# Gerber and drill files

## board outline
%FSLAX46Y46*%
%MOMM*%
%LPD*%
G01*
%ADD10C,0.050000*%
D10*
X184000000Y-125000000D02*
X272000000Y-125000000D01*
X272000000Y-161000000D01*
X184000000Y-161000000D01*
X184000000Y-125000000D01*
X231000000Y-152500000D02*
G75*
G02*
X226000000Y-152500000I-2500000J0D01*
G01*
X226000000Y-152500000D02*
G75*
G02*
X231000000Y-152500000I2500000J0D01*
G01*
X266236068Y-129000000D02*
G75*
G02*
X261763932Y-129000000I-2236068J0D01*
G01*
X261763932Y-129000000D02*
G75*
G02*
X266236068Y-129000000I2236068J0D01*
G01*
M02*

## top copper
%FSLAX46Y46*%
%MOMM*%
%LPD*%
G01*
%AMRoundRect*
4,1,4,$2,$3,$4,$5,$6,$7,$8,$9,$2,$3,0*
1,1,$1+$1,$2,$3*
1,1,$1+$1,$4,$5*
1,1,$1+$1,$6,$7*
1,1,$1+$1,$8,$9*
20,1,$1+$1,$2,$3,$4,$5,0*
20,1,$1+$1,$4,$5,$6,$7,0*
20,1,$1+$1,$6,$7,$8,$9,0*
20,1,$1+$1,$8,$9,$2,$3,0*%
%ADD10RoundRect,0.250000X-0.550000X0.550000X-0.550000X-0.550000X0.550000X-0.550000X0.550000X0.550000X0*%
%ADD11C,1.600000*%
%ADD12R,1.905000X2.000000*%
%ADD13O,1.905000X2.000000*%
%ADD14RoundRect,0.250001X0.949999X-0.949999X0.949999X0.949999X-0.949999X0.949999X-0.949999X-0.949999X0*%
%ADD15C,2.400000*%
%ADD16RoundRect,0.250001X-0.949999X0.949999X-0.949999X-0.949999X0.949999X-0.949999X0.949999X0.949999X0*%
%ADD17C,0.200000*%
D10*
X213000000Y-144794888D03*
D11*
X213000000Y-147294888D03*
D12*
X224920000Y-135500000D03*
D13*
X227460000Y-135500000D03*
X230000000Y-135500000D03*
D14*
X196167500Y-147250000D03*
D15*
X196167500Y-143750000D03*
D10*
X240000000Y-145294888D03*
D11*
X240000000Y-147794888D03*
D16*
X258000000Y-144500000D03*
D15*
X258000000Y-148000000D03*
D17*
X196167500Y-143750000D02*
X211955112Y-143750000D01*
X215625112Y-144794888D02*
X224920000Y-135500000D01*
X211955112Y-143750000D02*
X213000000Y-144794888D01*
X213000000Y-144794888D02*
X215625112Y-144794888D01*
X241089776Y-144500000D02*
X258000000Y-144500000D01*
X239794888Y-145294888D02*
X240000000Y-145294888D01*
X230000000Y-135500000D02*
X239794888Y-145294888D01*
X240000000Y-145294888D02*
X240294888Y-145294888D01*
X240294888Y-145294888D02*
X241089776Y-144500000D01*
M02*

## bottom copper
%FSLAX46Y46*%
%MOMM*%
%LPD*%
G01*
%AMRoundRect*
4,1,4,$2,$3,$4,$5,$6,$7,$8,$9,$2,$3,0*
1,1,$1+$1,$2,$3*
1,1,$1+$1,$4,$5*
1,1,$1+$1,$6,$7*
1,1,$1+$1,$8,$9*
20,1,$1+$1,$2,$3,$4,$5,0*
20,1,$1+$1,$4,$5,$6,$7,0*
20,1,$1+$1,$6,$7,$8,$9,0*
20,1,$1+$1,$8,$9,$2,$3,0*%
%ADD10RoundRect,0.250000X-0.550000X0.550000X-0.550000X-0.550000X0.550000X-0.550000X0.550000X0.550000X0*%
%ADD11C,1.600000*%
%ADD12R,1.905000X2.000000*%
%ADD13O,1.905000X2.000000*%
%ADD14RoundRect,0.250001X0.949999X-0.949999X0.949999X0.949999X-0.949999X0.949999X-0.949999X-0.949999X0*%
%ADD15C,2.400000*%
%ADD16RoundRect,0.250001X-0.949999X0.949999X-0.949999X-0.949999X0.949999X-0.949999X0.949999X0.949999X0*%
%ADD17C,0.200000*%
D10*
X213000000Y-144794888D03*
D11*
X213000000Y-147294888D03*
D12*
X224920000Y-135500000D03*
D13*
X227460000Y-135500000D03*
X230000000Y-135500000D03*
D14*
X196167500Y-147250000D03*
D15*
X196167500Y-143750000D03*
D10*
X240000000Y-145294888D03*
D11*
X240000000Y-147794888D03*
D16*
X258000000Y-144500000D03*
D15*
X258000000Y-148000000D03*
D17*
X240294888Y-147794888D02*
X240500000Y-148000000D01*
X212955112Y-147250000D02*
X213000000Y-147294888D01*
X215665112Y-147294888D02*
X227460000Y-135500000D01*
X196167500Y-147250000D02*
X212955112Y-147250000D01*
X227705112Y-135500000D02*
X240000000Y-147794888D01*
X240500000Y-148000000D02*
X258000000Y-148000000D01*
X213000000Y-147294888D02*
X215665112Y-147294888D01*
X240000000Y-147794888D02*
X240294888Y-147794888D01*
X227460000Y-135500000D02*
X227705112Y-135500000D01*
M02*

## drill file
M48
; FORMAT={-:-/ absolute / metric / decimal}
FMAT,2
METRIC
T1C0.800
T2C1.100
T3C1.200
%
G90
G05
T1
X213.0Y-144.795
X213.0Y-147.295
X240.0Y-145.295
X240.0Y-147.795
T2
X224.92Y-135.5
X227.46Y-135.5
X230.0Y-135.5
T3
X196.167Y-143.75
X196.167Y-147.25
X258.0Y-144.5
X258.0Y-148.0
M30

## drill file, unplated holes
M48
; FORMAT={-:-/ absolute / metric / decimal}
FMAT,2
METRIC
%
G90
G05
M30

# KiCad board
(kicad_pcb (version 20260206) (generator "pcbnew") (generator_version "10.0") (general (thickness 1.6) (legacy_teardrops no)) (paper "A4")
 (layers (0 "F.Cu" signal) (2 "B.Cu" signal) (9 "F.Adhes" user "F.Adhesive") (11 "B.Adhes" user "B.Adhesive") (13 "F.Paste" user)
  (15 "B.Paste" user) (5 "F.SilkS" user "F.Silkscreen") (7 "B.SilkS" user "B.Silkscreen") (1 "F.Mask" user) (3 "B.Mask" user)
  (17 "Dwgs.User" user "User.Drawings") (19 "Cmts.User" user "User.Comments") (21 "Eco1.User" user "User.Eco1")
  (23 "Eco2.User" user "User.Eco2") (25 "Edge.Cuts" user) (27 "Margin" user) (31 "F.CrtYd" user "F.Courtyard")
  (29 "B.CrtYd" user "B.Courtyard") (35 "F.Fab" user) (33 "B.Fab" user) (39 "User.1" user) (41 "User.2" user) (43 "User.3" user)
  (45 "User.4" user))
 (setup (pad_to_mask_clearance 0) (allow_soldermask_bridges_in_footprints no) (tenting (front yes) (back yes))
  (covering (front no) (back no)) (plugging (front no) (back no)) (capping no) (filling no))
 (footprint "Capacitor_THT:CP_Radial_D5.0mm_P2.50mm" (layer "F.Cu") (at 213 144.794888 -90)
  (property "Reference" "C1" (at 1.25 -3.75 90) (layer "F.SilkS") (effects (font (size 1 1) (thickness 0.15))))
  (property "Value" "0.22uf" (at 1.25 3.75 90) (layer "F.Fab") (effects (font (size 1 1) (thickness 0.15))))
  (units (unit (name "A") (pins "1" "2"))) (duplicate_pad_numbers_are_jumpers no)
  (pad "1" thru_hole roundrect (at 0 0 270) (size 1.6 1.6) (drill 0.8) (layers "*.Cu" "*.Mask") (remove_unused_layers no)
   (roundrect_rratio 0.15625) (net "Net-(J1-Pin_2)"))
  (pad "2" thru_hole circle (at 2.5 0 270) (size 1.6 1.6) (drill 0.8) (layers "*.Cu" "*.Mask") (remove_unused_layers no) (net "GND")))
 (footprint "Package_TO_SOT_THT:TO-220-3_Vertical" (layer "F.Cu") (at 224.92 135.5)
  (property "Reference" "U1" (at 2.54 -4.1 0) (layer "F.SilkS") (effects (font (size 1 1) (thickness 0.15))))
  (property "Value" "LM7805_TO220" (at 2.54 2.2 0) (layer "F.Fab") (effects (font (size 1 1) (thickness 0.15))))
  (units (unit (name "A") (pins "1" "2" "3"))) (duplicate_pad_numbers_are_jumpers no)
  (pad "1" thru_hole rect (at 0 0) (size 1.905 2) (drill 1.1) (layers "*.Cu" "*.Mask") (remove_unused_layers no) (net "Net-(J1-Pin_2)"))
  (pad "2" thru_hole oval (at 2.54 0) (size 1.905 2) (drill 1.1) (layers "*.Cu" "*.Mask") (remove_unused_layers no) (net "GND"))
  (pad "3" thru_hole oval (at 5.08 0) (size 1.905 2) (drill 1.1) (layers "*.Cu" "*.Mask") (remove_unused_layers no) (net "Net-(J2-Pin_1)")))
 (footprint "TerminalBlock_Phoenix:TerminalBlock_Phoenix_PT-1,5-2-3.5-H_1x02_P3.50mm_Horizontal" (layer "F.Cu") (at 196.1675 147.25 90)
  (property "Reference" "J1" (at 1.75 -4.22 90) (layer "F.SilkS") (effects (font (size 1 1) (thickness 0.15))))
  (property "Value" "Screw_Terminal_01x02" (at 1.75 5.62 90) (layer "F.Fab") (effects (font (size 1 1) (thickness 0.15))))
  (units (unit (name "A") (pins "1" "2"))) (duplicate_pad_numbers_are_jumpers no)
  (pad "1" thru_hole roundrect (at 0 0 90) (size 2.4 2.4) (drill 1.2) (layers "*.Cu" "*.Mask") (remove_unused_layers no)
   (roundrect_rratio 0.104167) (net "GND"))
  (pad "2" thru_hole circle (at 3.5 0 90) (size 2.4 2.4) (drill 1.2) (layers "*.Cu" "*.Mask") (remove_unused_layers no)
   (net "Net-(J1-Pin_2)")))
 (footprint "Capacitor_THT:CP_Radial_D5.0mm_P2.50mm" (layer "F.Cu") (at 240 145.294888 -90)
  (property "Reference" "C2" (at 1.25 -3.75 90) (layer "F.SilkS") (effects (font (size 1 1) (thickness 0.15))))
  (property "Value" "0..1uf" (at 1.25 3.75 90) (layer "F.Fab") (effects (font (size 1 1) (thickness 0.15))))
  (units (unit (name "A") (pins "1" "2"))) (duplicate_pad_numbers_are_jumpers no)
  (pad "1" thru_hole roundrect (at 0 0 270) (size 1.6 1.6) (drill 0.8) (layers "*.Cu" "*.Mask") (remove_unused_layers no)
   (roundrect_rratio 0.15625) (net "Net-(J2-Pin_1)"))
  (pad "2" thru_hole circle (at 2.5 0 270) (size 1.6 1.6) (drill 0.8) (layers "*.Cu" "*.Mask") (remove_unused_layers no) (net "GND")))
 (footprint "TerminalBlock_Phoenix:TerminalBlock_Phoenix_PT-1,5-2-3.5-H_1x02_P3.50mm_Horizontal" (layer "F.Cu") (at 258 144.5 -90)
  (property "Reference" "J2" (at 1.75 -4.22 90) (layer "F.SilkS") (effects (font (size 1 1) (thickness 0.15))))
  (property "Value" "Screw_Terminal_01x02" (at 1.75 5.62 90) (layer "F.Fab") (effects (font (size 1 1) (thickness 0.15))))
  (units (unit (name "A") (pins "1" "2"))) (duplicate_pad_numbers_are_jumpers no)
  (pad "1" thru_hole roundrect (at 0 0 270) (size 2.4 2.4) (drill 1.2) (layers "*.Cu" "*.Mask") (remove_unused_layers no)
   (roundrect_rratio 0.104167) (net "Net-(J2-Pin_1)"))
  (pad "2" thru_hole circle (at 3.5 0 270) (size 2.4 2.4) (drill 1.2) (layers "*.Cu" "*.Mask") (remove_unused_layers no) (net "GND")))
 (gr_rect (start 184 125) (end 272 161) (stroke (width 0.05) (type default)) (fill no) (layer "Edge.Cuts"))
 (gr_circle (center 228.5 152.5) (end 227 154.5) (stroke (width 0.05) (type default)) (fill no) (layer "Edge.Cuts"))
 (gr_circle (center 264 129) (end 263 131) (stroke (width 0.05) (type default)) (fill no) (layer "Edge.Cuts"))
 (segment (start 196.1675 143.75) (end 211.955112 143.75) (width 0.2) (layer "F.Cu") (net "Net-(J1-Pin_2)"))
 (segment (start 215.625112 144.794888) (end 224.92 135.5) (width 0.2) (layer "F.Cu") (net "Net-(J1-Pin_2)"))
 (segment (start 211.955112 143.75) (end 213 144.794888) (width 0.2) (layer "F.Cu") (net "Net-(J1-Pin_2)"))
 (segment (start 213 144.794888) (end 215.625112 144.794888) (width 0.2) (layer "F.Cu") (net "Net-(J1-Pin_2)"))
 (segment (start 240.294888 147.794888) (end 240.5 148) (width 0.2) (layer "B.Cu") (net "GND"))
 (segment (start 212.955112 147.25) (end 213 147.294888) (width 0.2) (layer "B.Cu") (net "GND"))
 (segment (start 215.665112 147.294888) (end 227.46 135.5) (width 0.2) (layer "B.Cu") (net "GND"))
 (segment (start 196.1675 147.25) (end 212.955112 147.25) (width 0.2) (layer "B.Cu") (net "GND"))
 (segment (start 227.705112 135.5) (end 240 147.794888) (width 0.2) (layer "B.Cu") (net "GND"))
 (segment (start 240.5 148) (end 258 148) (width 0.2) (layer "B.Cu") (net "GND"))
 (segment (start 213 147.294888) (end 215.665112 147.294888) (width 0.2) (layer "B.Cu") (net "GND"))
 (segment (start 240 147.794888) (end 240.294888 147.794888) (width 0.2) (layer "B.Cu") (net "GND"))
 (segment (start 227.46 135.5) (end 227.705112 135.5) (width 0.2) (layer "B.Cu") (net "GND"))
 (segment (start 241.089776 144.5) (end 258 144.5) (width 0.2) (layer "F.Cu") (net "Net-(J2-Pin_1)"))
 (segment (start 239.794888 145.294888) (end 240 145.294888) (width 0.2) (layer "F.Cu") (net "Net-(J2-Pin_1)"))
 (segment (start 230 135.5) (end 239.794888 145.294888) (width 0.2) (layer "F.Cu") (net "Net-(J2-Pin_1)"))
 (segment (start 240 145.294888) (end 240.294888 145.294888) (width 0.2) (layer "F.Cu") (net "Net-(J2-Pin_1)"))
 (segment (start 240.294888 145.294888) (end 241.089776 144.5) (width 0.2) (layer "F.Cu") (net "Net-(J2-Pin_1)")))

